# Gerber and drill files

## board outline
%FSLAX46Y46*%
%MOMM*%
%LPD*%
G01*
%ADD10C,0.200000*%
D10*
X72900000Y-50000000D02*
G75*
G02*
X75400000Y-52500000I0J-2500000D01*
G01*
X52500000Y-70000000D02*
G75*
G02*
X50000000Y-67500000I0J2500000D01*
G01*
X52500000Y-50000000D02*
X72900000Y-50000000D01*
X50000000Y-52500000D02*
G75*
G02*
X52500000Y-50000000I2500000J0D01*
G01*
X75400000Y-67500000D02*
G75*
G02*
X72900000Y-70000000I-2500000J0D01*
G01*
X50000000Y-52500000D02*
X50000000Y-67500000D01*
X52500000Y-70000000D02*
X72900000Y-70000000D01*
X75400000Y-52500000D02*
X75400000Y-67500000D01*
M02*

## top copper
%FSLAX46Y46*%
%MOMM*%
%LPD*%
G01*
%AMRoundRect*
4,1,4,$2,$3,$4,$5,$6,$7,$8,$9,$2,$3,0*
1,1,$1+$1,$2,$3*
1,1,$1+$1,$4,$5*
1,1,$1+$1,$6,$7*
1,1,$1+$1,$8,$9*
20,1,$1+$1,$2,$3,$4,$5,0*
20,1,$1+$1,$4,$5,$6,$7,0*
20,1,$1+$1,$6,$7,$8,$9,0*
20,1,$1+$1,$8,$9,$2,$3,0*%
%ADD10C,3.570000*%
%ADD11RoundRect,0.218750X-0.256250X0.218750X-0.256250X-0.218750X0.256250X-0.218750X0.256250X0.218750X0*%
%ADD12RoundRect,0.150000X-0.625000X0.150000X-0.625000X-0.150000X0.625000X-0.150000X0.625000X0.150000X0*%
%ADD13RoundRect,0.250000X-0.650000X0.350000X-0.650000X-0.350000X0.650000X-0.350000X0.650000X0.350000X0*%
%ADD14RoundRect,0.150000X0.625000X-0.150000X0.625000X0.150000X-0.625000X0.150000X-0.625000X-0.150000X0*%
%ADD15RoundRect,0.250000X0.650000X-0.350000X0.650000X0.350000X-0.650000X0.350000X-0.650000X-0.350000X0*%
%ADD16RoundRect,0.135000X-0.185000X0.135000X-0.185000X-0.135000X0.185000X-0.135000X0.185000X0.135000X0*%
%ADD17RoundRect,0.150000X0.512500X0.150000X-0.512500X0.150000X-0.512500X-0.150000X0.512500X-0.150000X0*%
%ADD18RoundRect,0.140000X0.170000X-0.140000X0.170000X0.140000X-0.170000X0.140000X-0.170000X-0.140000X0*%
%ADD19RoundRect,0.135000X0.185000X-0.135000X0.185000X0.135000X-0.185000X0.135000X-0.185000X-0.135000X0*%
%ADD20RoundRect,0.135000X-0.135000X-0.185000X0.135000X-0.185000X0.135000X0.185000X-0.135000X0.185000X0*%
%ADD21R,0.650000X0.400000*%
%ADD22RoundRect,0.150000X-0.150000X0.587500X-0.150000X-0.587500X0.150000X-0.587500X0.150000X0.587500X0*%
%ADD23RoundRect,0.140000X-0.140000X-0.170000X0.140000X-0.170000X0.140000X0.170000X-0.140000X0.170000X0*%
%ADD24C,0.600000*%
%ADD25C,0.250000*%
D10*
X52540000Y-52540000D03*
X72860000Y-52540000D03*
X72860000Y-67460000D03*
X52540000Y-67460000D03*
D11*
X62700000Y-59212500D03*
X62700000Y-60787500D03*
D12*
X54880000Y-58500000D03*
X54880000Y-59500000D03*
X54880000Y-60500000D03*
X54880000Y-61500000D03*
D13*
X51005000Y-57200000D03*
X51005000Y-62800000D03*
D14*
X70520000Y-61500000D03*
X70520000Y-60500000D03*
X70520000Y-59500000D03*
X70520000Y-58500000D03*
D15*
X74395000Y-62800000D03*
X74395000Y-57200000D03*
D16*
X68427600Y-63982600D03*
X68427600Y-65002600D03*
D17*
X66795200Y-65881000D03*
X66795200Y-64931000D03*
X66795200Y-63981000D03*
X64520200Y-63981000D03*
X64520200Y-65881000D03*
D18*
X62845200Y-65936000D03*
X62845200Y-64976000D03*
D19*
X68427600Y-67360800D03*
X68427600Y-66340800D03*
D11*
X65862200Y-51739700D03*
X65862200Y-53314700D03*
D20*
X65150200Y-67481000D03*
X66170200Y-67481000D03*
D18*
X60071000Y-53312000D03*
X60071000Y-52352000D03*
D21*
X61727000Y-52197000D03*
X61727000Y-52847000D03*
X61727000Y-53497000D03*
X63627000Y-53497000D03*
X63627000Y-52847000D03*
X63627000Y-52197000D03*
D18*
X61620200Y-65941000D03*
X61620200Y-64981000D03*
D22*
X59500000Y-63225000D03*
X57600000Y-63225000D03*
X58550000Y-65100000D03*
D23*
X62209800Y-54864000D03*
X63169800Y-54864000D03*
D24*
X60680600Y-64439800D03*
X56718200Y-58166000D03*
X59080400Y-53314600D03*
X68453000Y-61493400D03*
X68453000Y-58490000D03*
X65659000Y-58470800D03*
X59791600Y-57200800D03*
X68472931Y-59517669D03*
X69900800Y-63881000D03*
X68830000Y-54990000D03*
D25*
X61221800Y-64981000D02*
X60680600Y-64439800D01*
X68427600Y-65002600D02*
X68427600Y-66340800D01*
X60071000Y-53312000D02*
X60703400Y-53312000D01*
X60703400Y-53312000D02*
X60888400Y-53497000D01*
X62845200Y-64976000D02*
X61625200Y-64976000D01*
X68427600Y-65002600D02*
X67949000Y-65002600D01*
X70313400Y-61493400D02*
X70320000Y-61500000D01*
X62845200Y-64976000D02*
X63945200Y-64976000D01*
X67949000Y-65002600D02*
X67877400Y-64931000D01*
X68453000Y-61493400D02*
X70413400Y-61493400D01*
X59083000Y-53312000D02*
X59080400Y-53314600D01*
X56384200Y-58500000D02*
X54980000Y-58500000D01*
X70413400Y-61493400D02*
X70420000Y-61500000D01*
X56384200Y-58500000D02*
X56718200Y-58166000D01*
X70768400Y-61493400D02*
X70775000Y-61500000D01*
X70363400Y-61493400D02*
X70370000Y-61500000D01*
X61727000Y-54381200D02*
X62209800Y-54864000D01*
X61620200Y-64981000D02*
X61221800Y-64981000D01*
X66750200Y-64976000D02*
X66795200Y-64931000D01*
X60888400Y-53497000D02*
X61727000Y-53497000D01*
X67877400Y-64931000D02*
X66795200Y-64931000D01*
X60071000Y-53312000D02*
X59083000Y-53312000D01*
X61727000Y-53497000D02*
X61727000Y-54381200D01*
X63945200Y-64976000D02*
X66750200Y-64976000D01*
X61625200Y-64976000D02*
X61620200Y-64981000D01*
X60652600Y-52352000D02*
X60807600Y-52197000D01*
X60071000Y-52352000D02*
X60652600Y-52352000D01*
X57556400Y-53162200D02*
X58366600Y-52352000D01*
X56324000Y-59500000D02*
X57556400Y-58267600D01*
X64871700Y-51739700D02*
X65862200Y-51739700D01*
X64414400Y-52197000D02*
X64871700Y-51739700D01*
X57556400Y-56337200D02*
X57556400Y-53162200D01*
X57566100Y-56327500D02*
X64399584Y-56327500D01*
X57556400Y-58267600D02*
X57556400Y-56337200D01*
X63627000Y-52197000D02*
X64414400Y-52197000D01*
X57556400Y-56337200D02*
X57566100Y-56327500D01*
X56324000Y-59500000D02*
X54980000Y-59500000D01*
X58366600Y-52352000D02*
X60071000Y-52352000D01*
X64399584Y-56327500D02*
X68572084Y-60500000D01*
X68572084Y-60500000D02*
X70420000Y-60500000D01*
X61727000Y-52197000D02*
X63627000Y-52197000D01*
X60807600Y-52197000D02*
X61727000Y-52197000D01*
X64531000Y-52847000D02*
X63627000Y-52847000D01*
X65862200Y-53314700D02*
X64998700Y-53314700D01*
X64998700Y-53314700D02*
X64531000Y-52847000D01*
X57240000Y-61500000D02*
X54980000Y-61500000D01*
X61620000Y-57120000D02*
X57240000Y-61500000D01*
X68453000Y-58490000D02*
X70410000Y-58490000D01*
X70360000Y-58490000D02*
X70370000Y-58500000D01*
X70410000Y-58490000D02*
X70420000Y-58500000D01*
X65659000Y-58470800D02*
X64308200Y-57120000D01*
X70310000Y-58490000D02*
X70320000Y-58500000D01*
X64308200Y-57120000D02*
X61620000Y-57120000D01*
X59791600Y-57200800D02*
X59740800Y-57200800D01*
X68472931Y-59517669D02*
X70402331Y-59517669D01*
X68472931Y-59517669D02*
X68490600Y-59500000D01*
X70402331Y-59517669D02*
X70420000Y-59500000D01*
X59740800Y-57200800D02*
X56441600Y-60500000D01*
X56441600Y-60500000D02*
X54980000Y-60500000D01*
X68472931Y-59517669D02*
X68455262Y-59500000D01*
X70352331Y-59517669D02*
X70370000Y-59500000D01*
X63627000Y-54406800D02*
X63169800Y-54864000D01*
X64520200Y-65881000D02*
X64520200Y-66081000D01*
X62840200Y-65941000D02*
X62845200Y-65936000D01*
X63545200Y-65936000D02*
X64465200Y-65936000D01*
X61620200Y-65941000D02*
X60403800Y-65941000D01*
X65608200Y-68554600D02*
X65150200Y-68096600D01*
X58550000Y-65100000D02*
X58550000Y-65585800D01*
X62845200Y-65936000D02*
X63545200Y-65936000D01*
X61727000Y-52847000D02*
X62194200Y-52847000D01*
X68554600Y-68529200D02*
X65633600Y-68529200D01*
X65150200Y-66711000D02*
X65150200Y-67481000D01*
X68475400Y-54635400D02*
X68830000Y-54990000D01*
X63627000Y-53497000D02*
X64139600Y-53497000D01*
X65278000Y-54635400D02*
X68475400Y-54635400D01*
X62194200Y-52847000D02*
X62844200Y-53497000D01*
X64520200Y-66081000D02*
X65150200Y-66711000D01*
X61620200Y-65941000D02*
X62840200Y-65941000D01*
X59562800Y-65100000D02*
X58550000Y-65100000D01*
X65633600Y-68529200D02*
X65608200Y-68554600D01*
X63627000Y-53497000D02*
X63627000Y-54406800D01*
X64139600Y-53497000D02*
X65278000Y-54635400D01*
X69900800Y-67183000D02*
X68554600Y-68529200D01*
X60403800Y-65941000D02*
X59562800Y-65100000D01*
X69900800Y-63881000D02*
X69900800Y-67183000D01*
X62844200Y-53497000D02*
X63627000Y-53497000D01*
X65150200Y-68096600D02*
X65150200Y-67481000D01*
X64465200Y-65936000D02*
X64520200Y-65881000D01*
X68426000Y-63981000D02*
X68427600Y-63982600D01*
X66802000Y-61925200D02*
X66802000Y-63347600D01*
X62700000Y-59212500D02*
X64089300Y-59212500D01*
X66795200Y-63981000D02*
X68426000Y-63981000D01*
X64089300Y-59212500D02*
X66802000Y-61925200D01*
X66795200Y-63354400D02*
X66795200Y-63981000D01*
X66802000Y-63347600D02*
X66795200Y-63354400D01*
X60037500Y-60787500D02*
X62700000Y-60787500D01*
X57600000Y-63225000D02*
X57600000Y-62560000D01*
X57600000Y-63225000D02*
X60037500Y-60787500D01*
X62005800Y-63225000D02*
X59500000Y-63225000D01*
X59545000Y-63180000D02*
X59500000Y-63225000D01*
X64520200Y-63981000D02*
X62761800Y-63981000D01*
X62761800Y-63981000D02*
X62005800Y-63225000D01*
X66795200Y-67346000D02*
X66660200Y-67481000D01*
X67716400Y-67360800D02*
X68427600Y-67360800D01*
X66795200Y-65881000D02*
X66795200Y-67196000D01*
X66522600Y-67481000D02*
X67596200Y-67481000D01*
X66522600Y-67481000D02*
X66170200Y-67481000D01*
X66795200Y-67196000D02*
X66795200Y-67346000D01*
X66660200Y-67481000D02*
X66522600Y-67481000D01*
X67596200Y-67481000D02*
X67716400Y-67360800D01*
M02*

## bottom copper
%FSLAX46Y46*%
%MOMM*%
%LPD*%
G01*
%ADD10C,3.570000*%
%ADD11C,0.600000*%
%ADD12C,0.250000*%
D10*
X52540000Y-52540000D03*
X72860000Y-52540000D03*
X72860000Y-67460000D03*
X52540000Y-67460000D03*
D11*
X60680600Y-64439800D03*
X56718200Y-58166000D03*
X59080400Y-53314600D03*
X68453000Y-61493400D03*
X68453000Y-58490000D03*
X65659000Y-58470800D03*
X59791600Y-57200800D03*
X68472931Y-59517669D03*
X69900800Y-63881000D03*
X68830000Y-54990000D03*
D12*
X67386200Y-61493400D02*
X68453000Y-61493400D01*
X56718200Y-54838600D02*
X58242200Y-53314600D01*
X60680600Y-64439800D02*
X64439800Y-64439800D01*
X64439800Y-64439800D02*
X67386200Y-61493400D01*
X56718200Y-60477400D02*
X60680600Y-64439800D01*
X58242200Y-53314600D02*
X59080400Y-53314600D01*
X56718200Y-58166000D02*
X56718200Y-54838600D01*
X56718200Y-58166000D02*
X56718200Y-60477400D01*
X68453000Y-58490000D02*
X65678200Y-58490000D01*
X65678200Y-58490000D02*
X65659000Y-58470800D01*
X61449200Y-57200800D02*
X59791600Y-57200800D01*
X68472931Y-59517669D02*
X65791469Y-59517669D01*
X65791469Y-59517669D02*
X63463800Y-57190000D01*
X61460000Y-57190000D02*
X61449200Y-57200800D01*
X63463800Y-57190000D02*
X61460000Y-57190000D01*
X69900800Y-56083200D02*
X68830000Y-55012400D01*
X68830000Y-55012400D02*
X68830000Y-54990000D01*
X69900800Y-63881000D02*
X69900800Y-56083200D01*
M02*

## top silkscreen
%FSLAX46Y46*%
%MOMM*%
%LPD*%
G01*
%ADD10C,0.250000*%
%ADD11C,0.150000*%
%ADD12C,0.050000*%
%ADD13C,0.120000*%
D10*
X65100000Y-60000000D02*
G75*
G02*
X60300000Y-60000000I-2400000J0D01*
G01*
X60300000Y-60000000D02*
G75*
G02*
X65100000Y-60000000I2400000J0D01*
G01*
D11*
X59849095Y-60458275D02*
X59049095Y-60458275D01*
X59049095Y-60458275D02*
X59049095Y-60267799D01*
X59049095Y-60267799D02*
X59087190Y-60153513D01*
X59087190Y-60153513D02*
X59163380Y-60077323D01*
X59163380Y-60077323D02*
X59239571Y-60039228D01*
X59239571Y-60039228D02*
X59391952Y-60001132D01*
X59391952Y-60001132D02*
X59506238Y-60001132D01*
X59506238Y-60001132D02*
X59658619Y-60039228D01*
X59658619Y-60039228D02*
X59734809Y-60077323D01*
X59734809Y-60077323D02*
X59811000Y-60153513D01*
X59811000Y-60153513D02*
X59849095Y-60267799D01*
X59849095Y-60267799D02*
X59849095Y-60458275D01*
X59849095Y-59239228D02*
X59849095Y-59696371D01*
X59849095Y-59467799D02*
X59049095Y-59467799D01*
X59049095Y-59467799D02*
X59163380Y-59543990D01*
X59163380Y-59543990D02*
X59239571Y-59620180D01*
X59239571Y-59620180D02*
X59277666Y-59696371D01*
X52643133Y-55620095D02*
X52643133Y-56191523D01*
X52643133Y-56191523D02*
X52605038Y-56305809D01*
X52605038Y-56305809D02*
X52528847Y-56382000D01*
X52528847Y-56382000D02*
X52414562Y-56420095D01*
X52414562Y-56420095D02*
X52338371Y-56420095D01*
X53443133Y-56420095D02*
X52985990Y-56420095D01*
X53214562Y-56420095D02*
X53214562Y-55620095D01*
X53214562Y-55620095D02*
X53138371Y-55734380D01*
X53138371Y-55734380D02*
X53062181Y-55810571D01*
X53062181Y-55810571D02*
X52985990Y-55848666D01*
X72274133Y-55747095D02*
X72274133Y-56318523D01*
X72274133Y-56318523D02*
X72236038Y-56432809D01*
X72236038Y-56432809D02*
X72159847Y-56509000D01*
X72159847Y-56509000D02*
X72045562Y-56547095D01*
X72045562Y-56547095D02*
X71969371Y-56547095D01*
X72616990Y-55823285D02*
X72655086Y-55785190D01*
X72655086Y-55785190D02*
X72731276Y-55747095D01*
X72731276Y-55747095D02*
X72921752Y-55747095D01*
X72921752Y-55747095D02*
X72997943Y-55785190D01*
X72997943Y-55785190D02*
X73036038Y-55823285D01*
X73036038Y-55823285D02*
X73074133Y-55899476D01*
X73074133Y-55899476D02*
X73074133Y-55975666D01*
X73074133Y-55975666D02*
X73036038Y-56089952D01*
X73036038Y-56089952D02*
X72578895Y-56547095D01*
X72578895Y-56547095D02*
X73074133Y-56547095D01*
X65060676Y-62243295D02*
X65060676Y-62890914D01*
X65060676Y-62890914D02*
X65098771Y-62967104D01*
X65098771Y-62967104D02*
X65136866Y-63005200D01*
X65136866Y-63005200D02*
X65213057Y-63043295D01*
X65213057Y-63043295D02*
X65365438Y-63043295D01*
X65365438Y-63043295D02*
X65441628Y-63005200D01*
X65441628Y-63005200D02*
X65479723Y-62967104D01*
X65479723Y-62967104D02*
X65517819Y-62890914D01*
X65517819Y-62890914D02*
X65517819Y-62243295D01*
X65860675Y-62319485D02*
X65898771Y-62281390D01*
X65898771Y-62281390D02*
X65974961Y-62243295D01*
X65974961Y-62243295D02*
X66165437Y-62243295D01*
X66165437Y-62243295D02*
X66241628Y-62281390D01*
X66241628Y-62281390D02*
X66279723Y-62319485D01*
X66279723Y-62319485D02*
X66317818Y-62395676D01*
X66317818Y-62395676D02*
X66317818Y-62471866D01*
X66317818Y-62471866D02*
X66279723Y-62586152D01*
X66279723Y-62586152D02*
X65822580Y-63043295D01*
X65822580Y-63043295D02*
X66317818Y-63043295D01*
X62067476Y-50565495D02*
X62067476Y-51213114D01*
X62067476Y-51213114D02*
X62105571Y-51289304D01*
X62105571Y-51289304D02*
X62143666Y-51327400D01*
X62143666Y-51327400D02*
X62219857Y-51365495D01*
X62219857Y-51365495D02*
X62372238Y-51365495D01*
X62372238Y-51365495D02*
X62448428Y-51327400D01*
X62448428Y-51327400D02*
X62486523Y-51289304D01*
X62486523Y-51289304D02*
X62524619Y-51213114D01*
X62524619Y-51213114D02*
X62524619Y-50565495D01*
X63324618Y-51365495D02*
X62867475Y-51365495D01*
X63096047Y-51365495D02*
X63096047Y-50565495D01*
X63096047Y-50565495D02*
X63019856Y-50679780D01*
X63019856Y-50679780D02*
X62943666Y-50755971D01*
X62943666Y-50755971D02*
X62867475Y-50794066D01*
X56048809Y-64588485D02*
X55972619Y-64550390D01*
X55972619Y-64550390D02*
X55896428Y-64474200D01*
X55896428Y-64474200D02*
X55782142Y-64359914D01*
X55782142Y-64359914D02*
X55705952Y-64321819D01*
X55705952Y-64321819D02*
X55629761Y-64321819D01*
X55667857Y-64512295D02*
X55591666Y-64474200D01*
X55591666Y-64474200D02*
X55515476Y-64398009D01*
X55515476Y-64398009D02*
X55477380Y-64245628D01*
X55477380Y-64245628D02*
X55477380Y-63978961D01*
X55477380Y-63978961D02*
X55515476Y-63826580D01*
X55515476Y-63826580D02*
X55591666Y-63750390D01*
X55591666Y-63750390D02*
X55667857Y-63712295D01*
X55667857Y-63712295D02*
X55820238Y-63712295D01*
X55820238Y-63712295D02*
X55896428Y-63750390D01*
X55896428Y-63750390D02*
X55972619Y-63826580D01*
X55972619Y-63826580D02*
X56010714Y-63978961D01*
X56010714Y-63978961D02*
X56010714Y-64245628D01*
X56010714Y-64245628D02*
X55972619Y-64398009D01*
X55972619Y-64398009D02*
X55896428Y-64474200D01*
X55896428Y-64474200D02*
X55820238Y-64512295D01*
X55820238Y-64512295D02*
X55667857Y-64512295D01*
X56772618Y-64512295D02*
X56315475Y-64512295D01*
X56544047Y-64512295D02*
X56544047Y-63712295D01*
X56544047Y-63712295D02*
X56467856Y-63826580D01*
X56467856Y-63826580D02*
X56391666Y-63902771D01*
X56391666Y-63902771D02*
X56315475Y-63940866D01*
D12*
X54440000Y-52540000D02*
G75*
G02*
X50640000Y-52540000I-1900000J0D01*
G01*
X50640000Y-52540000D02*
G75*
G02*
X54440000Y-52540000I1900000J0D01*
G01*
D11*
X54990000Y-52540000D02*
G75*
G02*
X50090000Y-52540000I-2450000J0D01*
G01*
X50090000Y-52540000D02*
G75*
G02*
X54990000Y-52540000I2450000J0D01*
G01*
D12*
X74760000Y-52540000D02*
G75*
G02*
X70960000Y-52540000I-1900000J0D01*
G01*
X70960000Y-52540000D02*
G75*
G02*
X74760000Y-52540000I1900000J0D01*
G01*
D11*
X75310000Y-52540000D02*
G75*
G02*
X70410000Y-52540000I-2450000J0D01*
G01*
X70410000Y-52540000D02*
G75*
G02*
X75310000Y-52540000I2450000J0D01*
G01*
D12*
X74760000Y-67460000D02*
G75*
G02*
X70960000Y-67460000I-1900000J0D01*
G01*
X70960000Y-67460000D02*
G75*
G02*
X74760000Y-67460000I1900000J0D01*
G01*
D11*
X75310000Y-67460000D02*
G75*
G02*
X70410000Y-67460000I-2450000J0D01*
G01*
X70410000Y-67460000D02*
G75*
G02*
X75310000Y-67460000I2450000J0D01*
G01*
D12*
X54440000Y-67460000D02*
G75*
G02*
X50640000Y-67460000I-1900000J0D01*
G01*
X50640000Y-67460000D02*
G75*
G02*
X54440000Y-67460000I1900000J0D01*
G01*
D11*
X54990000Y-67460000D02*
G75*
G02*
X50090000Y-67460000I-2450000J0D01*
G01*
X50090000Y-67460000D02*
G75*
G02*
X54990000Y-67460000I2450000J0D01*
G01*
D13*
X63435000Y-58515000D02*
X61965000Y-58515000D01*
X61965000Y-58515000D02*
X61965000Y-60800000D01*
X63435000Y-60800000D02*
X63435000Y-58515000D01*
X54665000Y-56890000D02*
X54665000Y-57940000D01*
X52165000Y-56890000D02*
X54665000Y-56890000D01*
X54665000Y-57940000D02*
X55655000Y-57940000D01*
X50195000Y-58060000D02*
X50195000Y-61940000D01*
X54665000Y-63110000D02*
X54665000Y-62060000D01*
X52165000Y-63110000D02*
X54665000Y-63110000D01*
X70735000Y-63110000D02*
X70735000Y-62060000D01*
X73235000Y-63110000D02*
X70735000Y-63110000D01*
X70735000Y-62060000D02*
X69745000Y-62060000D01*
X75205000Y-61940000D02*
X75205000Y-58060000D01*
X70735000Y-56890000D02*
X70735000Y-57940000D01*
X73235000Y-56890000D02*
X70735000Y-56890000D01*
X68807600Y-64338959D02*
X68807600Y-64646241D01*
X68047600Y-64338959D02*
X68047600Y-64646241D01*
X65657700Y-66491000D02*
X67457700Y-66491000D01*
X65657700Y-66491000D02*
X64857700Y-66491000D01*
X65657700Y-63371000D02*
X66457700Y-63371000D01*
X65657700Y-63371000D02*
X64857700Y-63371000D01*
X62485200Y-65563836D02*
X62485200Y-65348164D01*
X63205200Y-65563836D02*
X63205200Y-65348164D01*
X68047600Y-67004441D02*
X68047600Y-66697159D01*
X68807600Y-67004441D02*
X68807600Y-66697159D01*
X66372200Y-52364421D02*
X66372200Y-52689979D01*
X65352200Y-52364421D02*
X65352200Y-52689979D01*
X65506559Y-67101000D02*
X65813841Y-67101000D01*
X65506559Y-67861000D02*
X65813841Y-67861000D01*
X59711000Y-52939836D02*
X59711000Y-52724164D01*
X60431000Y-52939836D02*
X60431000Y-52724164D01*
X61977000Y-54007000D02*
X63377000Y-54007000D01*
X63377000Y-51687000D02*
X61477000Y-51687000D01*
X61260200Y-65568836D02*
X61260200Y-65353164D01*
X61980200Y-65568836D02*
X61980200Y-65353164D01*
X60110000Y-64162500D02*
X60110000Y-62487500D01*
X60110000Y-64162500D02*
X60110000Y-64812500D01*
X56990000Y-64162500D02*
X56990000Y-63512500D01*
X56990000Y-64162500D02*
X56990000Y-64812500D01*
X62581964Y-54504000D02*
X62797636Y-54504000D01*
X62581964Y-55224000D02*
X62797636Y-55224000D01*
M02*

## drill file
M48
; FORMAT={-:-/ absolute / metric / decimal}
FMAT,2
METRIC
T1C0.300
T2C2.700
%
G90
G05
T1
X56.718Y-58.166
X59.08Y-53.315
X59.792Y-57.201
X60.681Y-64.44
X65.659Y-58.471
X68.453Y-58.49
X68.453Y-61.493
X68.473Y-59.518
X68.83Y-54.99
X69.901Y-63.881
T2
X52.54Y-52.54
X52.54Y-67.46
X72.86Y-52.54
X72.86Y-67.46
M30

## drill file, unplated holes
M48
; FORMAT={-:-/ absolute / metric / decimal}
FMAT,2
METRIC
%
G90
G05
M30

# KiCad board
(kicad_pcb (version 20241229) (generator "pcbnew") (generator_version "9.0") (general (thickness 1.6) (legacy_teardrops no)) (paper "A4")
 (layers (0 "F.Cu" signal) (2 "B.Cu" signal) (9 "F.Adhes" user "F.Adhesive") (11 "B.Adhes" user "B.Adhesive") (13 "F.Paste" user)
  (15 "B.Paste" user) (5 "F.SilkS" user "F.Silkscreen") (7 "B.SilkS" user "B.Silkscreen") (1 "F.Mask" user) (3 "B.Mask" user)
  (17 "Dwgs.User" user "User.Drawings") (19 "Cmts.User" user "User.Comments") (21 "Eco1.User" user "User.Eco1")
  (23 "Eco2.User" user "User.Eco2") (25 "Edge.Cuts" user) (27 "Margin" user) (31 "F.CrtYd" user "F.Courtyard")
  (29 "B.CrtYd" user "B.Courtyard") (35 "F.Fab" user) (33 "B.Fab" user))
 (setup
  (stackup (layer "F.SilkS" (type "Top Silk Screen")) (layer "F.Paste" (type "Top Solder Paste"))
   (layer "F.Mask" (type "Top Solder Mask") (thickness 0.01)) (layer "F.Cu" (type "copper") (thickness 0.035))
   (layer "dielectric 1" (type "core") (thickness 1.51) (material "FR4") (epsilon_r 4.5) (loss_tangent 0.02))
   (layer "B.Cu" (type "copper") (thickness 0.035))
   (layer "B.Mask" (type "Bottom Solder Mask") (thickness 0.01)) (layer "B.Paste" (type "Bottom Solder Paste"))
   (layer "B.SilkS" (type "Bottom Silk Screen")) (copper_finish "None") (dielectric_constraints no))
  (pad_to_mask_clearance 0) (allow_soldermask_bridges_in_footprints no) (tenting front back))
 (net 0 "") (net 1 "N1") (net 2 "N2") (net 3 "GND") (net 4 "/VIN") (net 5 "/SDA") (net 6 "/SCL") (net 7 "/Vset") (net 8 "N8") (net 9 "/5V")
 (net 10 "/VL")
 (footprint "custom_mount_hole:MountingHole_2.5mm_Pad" (layer "F.Cu") (at 52.54 52.54)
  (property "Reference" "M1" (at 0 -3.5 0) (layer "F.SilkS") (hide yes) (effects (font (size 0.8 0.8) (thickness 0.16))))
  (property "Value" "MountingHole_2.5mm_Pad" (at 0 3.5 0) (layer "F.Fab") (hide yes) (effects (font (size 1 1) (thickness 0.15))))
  (fp_circle (center 0 0) (end 1.9 0) (stroke (width 0.05) (type solid)) (fill no) (layer "F.SilkS"))
  (fp_circle (center 0 0) (end 2.45 0) (stroke (width 0.15) (type solid)) (fill no) (layer "F.SilkS"))
  (pad "~" thru_hole circle (at 0 0) (size 3.57 3.57) (drill 2.7) (layers "*.Cu" "*.Mask") (remove_unused_layers no)))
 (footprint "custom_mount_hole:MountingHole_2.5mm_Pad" (layer "F.Cu") (at 72.86 52.54)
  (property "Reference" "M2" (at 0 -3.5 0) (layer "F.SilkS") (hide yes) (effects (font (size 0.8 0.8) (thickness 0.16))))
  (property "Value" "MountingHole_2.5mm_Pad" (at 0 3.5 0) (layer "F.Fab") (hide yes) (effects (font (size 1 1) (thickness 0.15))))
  (fp_circle (center 0 0) (end 1.9 0) (stroke (width 0.05) (type solid)) (fill no) (layer "F.SilkS"))
  (fp_circle (center 0 0) (end 2.45 0) (stroke (width 0.15) (type solid)) (fill no) (layer "F.SilkS"))
  (pad "~" thru_hole circle (at 0 0) (size 3.57 3.57) (drill 2.7) (layers "*.Cu" "*.Mask") (remove_unused_layers no)))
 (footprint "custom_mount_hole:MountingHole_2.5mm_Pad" (layer "F.Cu") (at 72.86 67.46)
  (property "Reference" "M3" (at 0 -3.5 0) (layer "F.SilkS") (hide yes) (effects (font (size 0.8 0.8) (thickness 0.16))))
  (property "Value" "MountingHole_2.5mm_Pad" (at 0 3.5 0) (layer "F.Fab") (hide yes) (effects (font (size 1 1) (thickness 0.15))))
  (fp_circle (center 0 0) (end 1.9 0) (stroke (width 0.05) (type solid)) (fill no) (layer "F.SilkS"))
  (fp_circle (center 0 0) (end 2.45 0) (stroke (width 0.15) (type solid)) (fill no) (layer "F.SilkS"))
  (pad "~" thru_hole circle (at 0 0) (size 3.57 3.57) (drill 2.7) (layers "*.Cu" "*.Mask") (remove_unused_layers no)))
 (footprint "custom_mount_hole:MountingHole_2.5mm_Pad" (layer "F.Cu") (at 52.54 67.46)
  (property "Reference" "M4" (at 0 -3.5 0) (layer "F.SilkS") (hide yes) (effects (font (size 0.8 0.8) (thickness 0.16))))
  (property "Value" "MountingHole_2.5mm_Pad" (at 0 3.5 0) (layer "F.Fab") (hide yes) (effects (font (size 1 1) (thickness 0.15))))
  (fp_circle (center 0 0) (end 1.9 0) (stroke (width 0.05) (type solid)) (fill no) (layer "F.SilkS"))
  (fp_circle (center 0 0) (end 2.45 0) (stroke (width 0.15) (type solid)) (fill no) (layer "F.SilkS"))
  (pad "~" thru_hole circle (at 0 0) (size 3.57 3.57) (drill 2.7) (layers "*.Cu" "*.Mask") (remove_unused_layers no)))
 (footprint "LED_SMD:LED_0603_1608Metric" (layer "F.Cu") (at 62.7 60 -90)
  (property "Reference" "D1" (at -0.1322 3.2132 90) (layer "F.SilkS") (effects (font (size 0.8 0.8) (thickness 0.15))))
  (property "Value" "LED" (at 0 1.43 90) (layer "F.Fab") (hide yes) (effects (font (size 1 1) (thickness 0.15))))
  (fp_line (start -1.485 0.735) (end 0.8 0.735) (stroke (width 0.12) (type solid)) (layer "F.SilkS"))
  (fp_line (start -1.485 -0.735) (end -1.485 0.735) (stroke (width 0.12) (type solid)) (layer "F.SilkS"))
  (fp_line (start 0.8 -0.735) (end -1.485 -0.735) (stroke (width 0.12) (type solid)) (layer "F.SilkS"))
  (pad "1" smd roundrect (at -0.7875 0 270) (size 0.875 0.95) (layers "F.Cu" "F.Mask" "F.Paste") (roundrect_rratio 0.25) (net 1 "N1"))
  (pad "2" smd roundrect (at 0.7875 0 270) (size 0.875 0.95) (layers "F.Cu" "F.Mask" "F.Paste") (roundrect_rratio 0.25) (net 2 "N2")))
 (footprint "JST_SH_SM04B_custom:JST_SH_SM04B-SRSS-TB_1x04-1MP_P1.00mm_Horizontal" (layer "F.Cu") (at 52.88 60 -90)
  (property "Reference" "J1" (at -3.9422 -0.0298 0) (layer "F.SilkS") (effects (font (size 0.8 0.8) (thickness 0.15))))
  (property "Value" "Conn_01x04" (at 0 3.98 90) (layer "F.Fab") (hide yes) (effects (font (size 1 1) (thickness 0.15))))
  (fp_line (start -1.94 2.685) (end 1.94 2.685) (stroke (width 0.12) (type solid)) (layer "F.SilkS"))
  (fp_line (start -3.11 0.715) (end -3.11 -1.785) (stroke (width 0.12) (type solid)) (layer "F.SilkS"))
  (fp_line (start 3.11 0.715) (end 3.11 -1.785) (stroke (width 0.12) (type solid)) (layer "F.SilkS"))
  (fp_line (start -3.11 -1.785) (end -2.06 -1.785) (stroke (width 0.12) (type solid)) (layer "F.SilkS"))
  (fp_line (start -2.06 -1.785) (end -2.06 -2.775) (stroke (width 0.12) (type solid)) (layer "F.SilkS"))
  (fp_line (start 3.11 -1.785) (end 2.06 -1.785) (stroke (width 0.12) (type solid)) (layer "F.SilkS"))
  (pad "1" smd roundrect (at -1.5 -2 270) (size 0.6 1.55) (layers "F.Cu" "F.Mask" "F.Paste") (roundrect_rratio 0.25) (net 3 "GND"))
  (pad "2" smd roundrect (at -0.5 -2 270) (size 0.6 1.55) (layers "F.Cu" "F.Mask" "F.Paste") (roundrect_rratio 0.25) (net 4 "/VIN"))
  (pad "3" smd roundrect (at 0.5 -2 270) (size 0.6 1.55) (layers "F.Cu" "F.Mask" "F.Paste") (roundrect_rratio 0.25) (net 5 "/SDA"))
  (pad "4" smd roundrect (at 1.5 -2 270) (size 0.6 1.55) (layers "F.Cu" "F.Mask" "F.Paste") (roundrect_rratio 0.25) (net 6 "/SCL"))
  (pad "MP" smd roundrect (at -2.8 1.875 270) (size 1.2 1.8) (layers "F.Cu" "F.Mask" "F.Paste") (roundrect_rratio 0.2083333333))
  (pad "MP" smd roundrect (at 2.8 1.875 270) (size 1.2 1.8) (layers "F.Cu" "F.Mask" "F.Paste") (roundrect_rratio 0.2083333333)))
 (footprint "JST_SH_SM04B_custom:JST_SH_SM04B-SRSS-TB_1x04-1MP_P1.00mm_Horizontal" (layer "F.Cu") (at 72.52 60 90)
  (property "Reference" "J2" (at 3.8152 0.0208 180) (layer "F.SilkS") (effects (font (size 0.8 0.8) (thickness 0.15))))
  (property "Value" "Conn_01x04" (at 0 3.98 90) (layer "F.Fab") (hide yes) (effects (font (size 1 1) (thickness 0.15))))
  (fp_line (start 3.11 -1.785) (end 2.06 -1.785) (stroke (width 0.12) (type solid)) (layer "F.SilkS"))
  (fp_line (start -2.06 -1.785) (end -2.06 -2.775) (stroke (width 0.12) (type solid)) (layer "F.SilkS"))
  (fp_line (start -3.11 -1.785) (end -2.06 -1.785) (stroke (width 0.12) (type solid)) (layer "F.SilkS"))
  (fp_line (start 3.11 0.715) (end 3.11 -1.785) (stroke (width 0.12) (type solid)) (layer "F.SilkS"))
  (fp_line (start -3.11 0.715) (end -3.11 -1.785) (stroke (width 0.12) (type solid)) (layer "F.SilkS"))
  (fp_line (start -1.94 2.685) (end 1.94 2.685) (stroke (width 0.12) (type solid)) (layer "F.SilkS"))
  (pad "1" smd roundrect (at -1.5 -2 90) (size 0.6 1.55) (layers "F.Cu" "F.Mask" "F.Paste") (roundrect_rratio 0.25) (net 3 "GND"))
  (pad "2" smd roundrect (at -0.5 -2 90) (size 0.6 1.55) (layers "F.Cu" "F.Mask" "F.Paste") (roundrect_rratio 0.25) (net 4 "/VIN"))
  (pad "3" smd roundrect (at 0.5 -2 90) (size 0.6 1.55) (layers "F.Cu" "F.Mask" "F.Paste") (roundrect_rratio 0.25) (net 5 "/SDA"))
  (pad "4" smd roundrect (at 1.5 -2 90) (size 0.6 1.55) (layers "F.Cu" "F.Mask" "F.Paste") (roundrect_rratio 0.25) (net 6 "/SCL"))
  (pad "MP" smd roundrect (at -2.8 1.875 90) (size 1.2 1.8) (layers "F.Cu" "F.Mask" "F.Paste") (roundrect_rratio 0.2083333333))
  (pad "MP" smd roundrect (at 2.8 1.875 90) (size 1.2 1.8) (layers "F.Cu" "F.Mask" "F.Paste") (roundrect_rratio 0.2083333333)))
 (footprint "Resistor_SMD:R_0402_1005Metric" (layer "F.Cu") (at 68.4276 64.4926 -90)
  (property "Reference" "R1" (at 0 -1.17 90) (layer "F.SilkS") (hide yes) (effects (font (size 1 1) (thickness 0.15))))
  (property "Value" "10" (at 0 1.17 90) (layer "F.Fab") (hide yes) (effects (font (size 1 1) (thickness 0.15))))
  (fp_line (start -0.153641 0.38) (end 0.153641 0.38) (stroke (width 0.12) (type solid)) (layer "F.SilkS"))
  (fp_line (start -0.153641 -0.38) (end 0.153641 -0.38) (stroke (width 0.12) (type solid)) (layer "F.SilkS"))
  (pad "1" smd roundrect (at -0.51 0 270) (size 0.54 0.64) (layers "F.Cu" "F.Mask" "F.Paste") (roundrect_rratio 0.25) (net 1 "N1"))
  (pad "2" smd roundrect (at 0.51 0 270) (size 0.54 0.64) (layers "F.Cu" "F.Mask" "F.Paste") (roundrect_rratio 0.25) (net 3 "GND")))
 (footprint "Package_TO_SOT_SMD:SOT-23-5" (layer "F.Cu") (at 65.6577 64.931 180)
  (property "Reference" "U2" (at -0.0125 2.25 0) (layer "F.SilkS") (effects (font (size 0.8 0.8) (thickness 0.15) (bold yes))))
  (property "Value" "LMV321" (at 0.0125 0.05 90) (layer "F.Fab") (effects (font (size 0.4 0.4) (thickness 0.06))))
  (fp_line (start 0 1.56) (end 0.8 1.56) (stroke (width 0.12) (type solid)) (layer "F.SilkS"))
  (fp_line (start 0 1.56) (end -0.8 1.56) (stroke (width 0.12) (type solid)) (layer "F.SilkS"))
  (fp_line (start 0 -1.56) (end 0.8 -1.56) (stroke (width 0.12) (type solid)) (layer "F.SilkS"))
  (fp_line (start 0 -1.56) (end -1.8 -1.56) (stroke (width 0.12) (type solid)) (layer "F.SilkS"))
  (pad "1" smd roundrect (at -1.1375 -0.95 180) (size 1.325 0.6) (layers "F.Cu" "F.Mask" "F.Paste") (roundrect_rratio 0.25) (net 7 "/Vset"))
  (pad "2" smd roundrect (at -1.1375 0 180) (size 1.325 0.6) (layers "F.Cu" "F.Mask" "F.Paste") (roundrect_rratio 0.25) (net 3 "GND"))
  (pad "3" smd roundrect (at -1.1375 0.95 180) (size 1.325 0.6) (layers "F.Cu" "F.Mask" "F.Paste") (roundrect_rratio 0.25) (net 1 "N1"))
  (pad "4" smd roundrect (at 1.1375 0.95 180) (size 1.325 0.6) (layers "F.Cu" "F.Mask" "F.Paste") (roundrect_rratio 0.25) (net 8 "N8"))
  (pad "5" smd roundrect (at 1.1375 -0.95 180) (size 1.325 0.6) (layers "F.Cu" "F.Mask" "F.Paste") (roundrect_rratio 0.25) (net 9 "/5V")))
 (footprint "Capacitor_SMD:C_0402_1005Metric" (layer "F.Cu") (at 62.8452 65.456 90)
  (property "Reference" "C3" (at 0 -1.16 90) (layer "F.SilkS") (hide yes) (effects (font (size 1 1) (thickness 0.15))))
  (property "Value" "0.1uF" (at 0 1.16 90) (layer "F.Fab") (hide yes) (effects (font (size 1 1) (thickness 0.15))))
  (fp_line (start -0.107836 -0.36) (end 0.107836 -0.36) (stroke (width 0.12) (type solid)) (layer "F.SilkS"))
  (fp_line (start -0.107836 0.36) (end 0.107836 0.36) (stroke (width 0.12) (type solid)) (layer "F.SilkS"))
  (pad "1" smd roundrect (at -0.48 0 90) (size 0.56 0.62) (layers "F.Cu" "F.Mask" "F.Paste") (roundrect_rratio 0.25) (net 9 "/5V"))
  (pad "2" smd roundrect (at 0.48 0 90) (size 0.56 0.62) (layers "F.Cu" "F.Mask" "F.Paste") (roundrect_rratio 0.25) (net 3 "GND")))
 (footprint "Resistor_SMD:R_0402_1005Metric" (layer "F.Cu") (at 68.4276 66.8508 90)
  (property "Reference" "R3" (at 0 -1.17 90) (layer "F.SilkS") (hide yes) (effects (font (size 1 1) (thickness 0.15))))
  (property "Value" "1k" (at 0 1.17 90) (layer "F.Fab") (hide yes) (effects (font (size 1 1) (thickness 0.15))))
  (fp_line (start -0.153641 -0.38) (end 0.153641 -0.38) (stroke (width 0.12) (type solid)) (layer "F.SilkS"))
  (fp_line (start -0.153641 0.38) (end 0.153641 0.38) (stroke (width 0.12) (type solid)) (layer "F.SilkS"))
  (pad "1" smd roundrect (at -0.51 0 90) (size 0.54 0.64) (layers "F.Cu" "F.Mask" "F.Paste") (roundrect_rratio 0.25) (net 7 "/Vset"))
  (pad "2" smd roundrect (at 0.51 0 90) (size 0.54 0.64) (layers "F.Cu" "F.Mask" "F.Paste") (roundrect_rratio 0.25) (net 3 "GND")))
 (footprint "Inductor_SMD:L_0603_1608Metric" (layer "F.Cu") (at 65.8622 52.5272 -90)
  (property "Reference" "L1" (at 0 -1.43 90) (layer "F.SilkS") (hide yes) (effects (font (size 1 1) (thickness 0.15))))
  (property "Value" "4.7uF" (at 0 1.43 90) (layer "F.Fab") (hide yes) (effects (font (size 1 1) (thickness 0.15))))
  (fp_line (start -0.162779 0.51) (end 0.162779 0.51) (stroke (width 0.12) (type solid)) (layer "F.SilkS"))
  (fp_line (start -0.162779 -0.51) (end 0.162779 -0.51) (stroke (width 0.12) (type solid)) (layer "F.SilkS"))
  (pad "1" smd roundrect (at -0.7875 0 270) (size 0.875 0.95) (layers "F.Cu" "F.Mask" "F.Paste") (roundrect_rratio 0.25) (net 4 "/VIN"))
  (pad "2" smd roundrect (at 0.7875 0 270) (size 0.875 0.95) (layers "F.Cu" "F.Mask" "F.Paste") (roundrect_rratio 0.25) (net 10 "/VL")))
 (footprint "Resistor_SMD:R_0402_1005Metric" (layer "F.Cu") (at 65.6602 67.481)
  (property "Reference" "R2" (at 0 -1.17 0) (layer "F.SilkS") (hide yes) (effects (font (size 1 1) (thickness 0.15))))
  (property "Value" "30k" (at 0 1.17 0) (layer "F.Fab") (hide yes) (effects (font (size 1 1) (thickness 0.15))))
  (fp_line (start -0.153641 -0.38) (end 0.153641 -0.38) (stroke (width 0.12) (type solid)) (layer "F.SilkS"))
  (fp_line (start -0.153641 0.38) (end 0.153641 0.38) (stroke (width 0.12) (type solid)) (layer "F.SilkS"))
  (pad "1" smd roundrect (at -0.51 0) (size 0.54 0.64) (layers "F.Cu" "F.Mask" "F.Paste") (roundrect_rratio 0.25) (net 9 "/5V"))
  (pad "2" smd roundrect (at 0.51 0) (size 0.54 0.64) (layers "F.Cu" "F.Mask" "F.Paste") (roundrect_rratio 0.25) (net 7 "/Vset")))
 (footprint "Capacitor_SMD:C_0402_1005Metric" (layer "F.Cu") (at 60.071 52.832 90)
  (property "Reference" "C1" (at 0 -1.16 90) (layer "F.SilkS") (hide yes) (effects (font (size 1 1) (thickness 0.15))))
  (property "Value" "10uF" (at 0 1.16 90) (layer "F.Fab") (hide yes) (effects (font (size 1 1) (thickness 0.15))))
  (fp_line (start -0.107836 -0.36) (end 0.107836 -0.36) (stroke (width 0.12) (type solid)) (layer "F.SilkS"))
  (fp_line (start -0.107836 0.36) (end 0.107836 0.36) (stroke (width 0.12) (type solid)) (layer "F.SilkS"))
  (pad "1" smd roundrect (at -0.48 0 90) (size 0.56 0.62) (layers "F.Cu" "F.Mask" "F.Paste") (roundrect_rratio 0.25) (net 3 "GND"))
  (pad "2" smd roundrect (at 0.48 0 90) (size 0.56 0.62) (layers "F.Cu" "F.Mask" "F.Paste") (roundrect_rratio 0.25) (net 4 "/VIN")))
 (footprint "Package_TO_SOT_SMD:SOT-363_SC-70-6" (layer "F.Cu") (at 62.677 52.847)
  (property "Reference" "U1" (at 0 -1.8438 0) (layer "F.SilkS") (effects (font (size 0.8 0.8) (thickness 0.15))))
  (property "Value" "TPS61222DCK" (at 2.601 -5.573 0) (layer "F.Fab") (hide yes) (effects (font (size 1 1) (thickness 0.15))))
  (fp_line (start -0.7 1.16) (end 0.7 1.16) (stroke (width 0.12) (type solid)) (layer "F.SilkS"))
  (fp_line (start 0.7 -1.16) (end -1.2 -1.16) (stroke (width 0.12) (type solid)) (layer "F.SilkS"))
  (pad "1" smd rect (at -0.95 -0.65) (size 0.65 0.4) (layers "F.Cu" "F.Mask" "F.Paste") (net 4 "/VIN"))
  (pad "2" smd rect (at -0.95 0) (size 0.65 0.4) (layers "F.Cu" "F.Mask" "F.Paste") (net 9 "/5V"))
  (pad "3" smd rect (at -0.95 0.65) (size 0.65 0.4) (layers "F.Cu" "F.Mask" "F.Paste") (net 3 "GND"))
  (pad "4" smd rect (at 0.95 0.65) (size 0.65 0.4) (layers "F.Cu" "F.Mask" "F.Paste") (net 9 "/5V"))
  (pad "5" smd rect (at 0.95 0) (size 0.65 0.4) (layers "F.Cu" "F.Mask" "F.Paste") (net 10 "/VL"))
  (pad "6" smd rect (at 0.95 -0.65) (size 0.65 0.4) (layers "F.Cu" "F.Mask" "F.Paste") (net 4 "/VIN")))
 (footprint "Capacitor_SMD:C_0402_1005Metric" (layer "F.Cu") (at 61.6202 65.461 90)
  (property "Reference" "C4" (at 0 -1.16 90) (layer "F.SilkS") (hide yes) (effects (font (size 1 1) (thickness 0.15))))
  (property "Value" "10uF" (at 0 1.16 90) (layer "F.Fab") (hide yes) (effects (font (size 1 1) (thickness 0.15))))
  (fp_line (start -0.107836 -0.36) (end 0.107836 -0.36) (stroke (width 0.12) (type solid)) (layer "F.SilkS"))
  (fp_line (start -0.107836 0.36) (end 0.107836 0.36) (stroke (width 0.12) (type solid)) (layer "F.SilkS"))
  (pad "1" smd roundrect (at -0.48 0 90) (size 0.56 0.62) (layers "F.Cu" "F.Mask" "F.Paste") (roundrect_rratio 0.25) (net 9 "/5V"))
  (pad "2" smd roundrect (at 0.48 0 90) (size 0.56 0.62) (layers "F.Cu" "F.Mask" "F.Paste") (roundrect_rratio 0.25) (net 3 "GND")))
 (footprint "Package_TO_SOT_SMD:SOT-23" (layer "F.Cu") (at 58.55 64.1625 -90)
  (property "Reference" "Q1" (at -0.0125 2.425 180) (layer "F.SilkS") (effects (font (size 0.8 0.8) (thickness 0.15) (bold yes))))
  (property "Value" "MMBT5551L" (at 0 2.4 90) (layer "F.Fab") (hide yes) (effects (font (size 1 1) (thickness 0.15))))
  (fp_line (start 0 1.56) (end -0.65 1.56) (stroke (width 0.12) (type solid)) (layer "F.SilkS"))
  (fp_line (start 0 1.56) (end 0.65 1.56) (stroke (width 0.12) (type solid)) (layer "F.SilkS"))
  (fp_line (start 0 -1.56) (end -1.675 -1.56) (stroke (width 0.12) (type solid)) (layer "F.SilkS"))
  (fp_line (start 0 -1.56) (end 0.65 -1.56) (stroke (width 0.12) (type solid)) (layer "F.SilkS"))
  (pad "1" smd roundrect (at -0.9375 -0.95 270) (size 1.475 0.6) (layers "F.Cu" "F.Mask" "F.Paste") (roundrect_rratio 0.25) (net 8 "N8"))
  (pad "2" smd roundrect (at -0.9375 0.95 270) (size 1.475 0.6) (layers "F.Cu" "F.Mask" "F.Paste") (roundrect_rratio 0.25) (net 2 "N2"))
  (pad "3" smd roundrect (at 0.9375 0 270) (size 1.475 0.6) (layers "F.Cu" "F.Mask" "F.Paste") (roundrect_rratio 0.25) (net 9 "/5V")))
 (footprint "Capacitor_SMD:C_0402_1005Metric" (layer "F.Cu") (at 62.6898 54.864)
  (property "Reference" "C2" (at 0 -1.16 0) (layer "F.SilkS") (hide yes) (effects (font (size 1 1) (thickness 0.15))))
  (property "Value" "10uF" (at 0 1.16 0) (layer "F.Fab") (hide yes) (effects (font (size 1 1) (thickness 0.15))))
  (fp_line (start -0.107836 -0.36) (end 0.107836 -0.36) (stroke (width 0.12) (type solid)) (layer "F.SilkS"))
  (fp_line (start -0.107836 0.36) (end 0.107836 0.36) (stroke (width 0.12) (type solid)) (layer "F.SilkS"))
  (pad "1" smd roundrect (at -0.48 0) (size 0.56 0.62) (layers "F.Cu" "F.Mask" "F.Paste") (roundrect_rratio 0.25) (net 3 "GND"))
  (pad "2" smd roundrect (at 0.48 0) (size 0.56 0.62) (layers "F.Cu" "F.Mask" "F.Paste") (roundrect_rratio 0.25) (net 9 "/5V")))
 (gr_circle (center 62.7 60) (end 65.1 60) (stroke (width 0.25) (type solid)) (fill no) (layer "F.SilkS"))
 (gr_arc (start 72.9 50) (mid 74.667767 50.732233) (end 75.4 52.5) (stroke (width 0.2) (type solid)) (layer "Edge.Cuts"))
 (gr_arc (start 52.5 70) (mid 50.732233 69.267767) (end 50 67.5) (stroke (width 0.2) (type solid)) (layer "Edge.Cuts"))
 (gr_line (start 52.5 50) (end 72.9 50) (stroke (width 0.2) (type solid)) (layer "Edge.Cuts"))
 (gr_arc (start 50 52.5) (mid 50.732233 50.732233) (end 52.5 50) (stroke (width 0.2) (type solid)) (layer "Edge.Cuts"))
 (gr_arc (start 75.4 67.5) (mid 74.667767 69.267767) (end 72.9 70) (stroke (width 0.2) (type solid)) (layer "Edge.Cuts"))
 (gr_line (start 50 52.5) (end 50 67.5) (stroke (width 0.2) (type solid)) (layer "Edge.Cuts"))
 (gr_line (start 52.5 70) (end 72.9 70) (stroke (width 0.2) (type solid)) (layer "Edge.Cuts"))
 (gr_line (start 75.4 52.5) (end 75.4 67.5) (stroke (width 0.2) (type solid)) (layer "Edge.Cuts"))
 (segment (start 61.2218 64.981) (end 60.6806 64.4398) (width 0.25) (layer "F.Cu") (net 3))
 (segment (start 68.4276 65.0026) (end 68.4276 66.3408) (width 0.25) (layer "F.Cu") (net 3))
 (segment (start 60.071 53.312) (end 60.7034 53.312) (width 0.25) (layer "F.Cu") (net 3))
 (segment (start 60.7034 53.312) (end 60.8884 53.497) (width 0.25) (layer "F.Cu") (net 3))
 (segment (start 62.8452 64.976) (end 61.6252 64.976) (width 0.25) (layer "F.Cu") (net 3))
 (segment (start 68.4276 65.0026) (end 67.949 65.0026) (width 0.25) (layer "F.Cu") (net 3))
 (segment (start 70.3134 61.4934) (end 70.32 61.5) (width 0.25) (layer "F.Cu") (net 3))
 (segment (start 62.8452 64.976) (end 63.9452 64.976) (width 0.25) (layer "F.Cu") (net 3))
 (segment (start 67.949 65.0026) (end 67.8774 64.931) (width 0.25) (layer "F.Cu") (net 3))
 (segment (start 68.453 61.4934) (end 70.4134 61.4934) (width 0.25) (layer "F.Cu") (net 3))
 (segment (start 59.083 53.312) (end 59.0804 53.3146) (width 0.25) (layer "F.Cu") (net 3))
 (segment (start 56.3842 58.5) (end 54.98 58.5) (width 0.25) (layer "F.Cu") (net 3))
 (segment (start 70.4134 61.4934) (end 70.42 61.5) (width 0.25) (layer "F.Cu") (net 3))
 (segment (start 56.3842 58.5) (end 56.7182 58.166) (width 0.25) (layer "F.Cu") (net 3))
 (segment (start 70.7684 61.4934) (end 70.775 61.5) (width 0.25) (layer "F.Cu") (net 3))
 (segment (start 70.3634 61.4934) (end 70.37 61.5) (width 0.25) (layer "F.Cu") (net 3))
 (segment (start 61.727 54.3812) (end 62.2098 54.864) (width 0.25) (layer "F.Cu") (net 3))
 (segment (start 61.6202 64.981) (end 61.2218 64.981) (width 0.25) (layer "F.Cu") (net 3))
 (segment (start 66.7502 64.976) (end 66.7952 64.931) (width 0.25) (layer "F.Cu") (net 3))
 (segment (start 60.8884 53.497) (end 61.727 53.497) (width 0.25) (layer "F.Cu") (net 3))
 (segment (start 67.8774 64.931) (end 66.7952 64.931) (width 0.25) (layer "F.Cu") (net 3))
 (segment (start 60.071 53.312) (end 59.083 53.312) (width 0.25) (layer "F.Cu") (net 3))
 (segment (start 61.727 53.497) (end 61.727 54.3812) (width 0.25) (layer "F.Cu") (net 3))
 (segment (start 63.9452 64.976) (end 66.7502 64.976) (width 0.25) (layer "F.Cu") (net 3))
 (segment (start 61.6252 64.976) (end 61.6202 64.981) (width 0.25) (layer "F.Cu") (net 3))
 (via (at 60.6806 64.4398) (size 0.6) (drill 0.3) (layers "F.Cu" "B.Cu") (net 3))
 (via (at 56.7182 58.166) (size 0.6) (drill 0.3) (layers "F.Cu" "B.Cu") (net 3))
 (via (at 59.0804 53.3146) (size 0.6) (drill 0.3) (layers "F.Cu" "B.Cu") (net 3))
 (via (at 68.453 61.4934) (size 0.6) (drill 0.3) (layers "F.Cu" "B.Cu") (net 3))
 (segment (start 67.3862 61.4934) (end 68.453 61.4934) (width 0.25) (layer "B.Cu") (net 3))
 (segment (start 56.7182 54.8386) (end 58.2422 53.3146) (width 0.25) (layer "B.Cu") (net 3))
 (segment (start 60.6806 64.4398) (end 64.4398 64.4398) (width 0.25) (layer "B.Cu") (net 3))
 (segment (start 64.4398 64.4398) (end 67.3862 61.4934) (width 0.25) (layer "B.Cu") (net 3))
 (segment (start 56.7182 60.4774) (end 60.6806 64.4398) (width 0.25) (layer "B.Cu") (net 3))
 (segment (start 58.2422 53.3146) (end 59.0804 53.3146) (width 0.25) (layer "B.Cu") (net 3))
 (segment (start 56.7182 58.166) (end 56.7182 54.8386) (width 0.25) (layer "B.Cu") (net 3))
 (segment (start 56.7182 58.166) (end 56.7182 60.4774) (width 0.25) (layer "B.Cu") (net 3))
 (segment (start 60.6526 52.352) (end 60.8076 52.197) (width 0.25) (layer "F.Cu") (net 4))
 (segment (start 60.071 52.352) (end 60.6526 52.352) (width 0.25) (layer "F.Cu") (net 4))
 (segment (start 57.5564 53.1622) (end 58.3666 52.352) (width 0.25) (layer "F.Cu") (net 4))
 (segment (start 56.324 59.5) (end 57.5564 58.2676) (width 0.25) (layer "F.Cu") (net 4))
 (segment (start 64.8717 51.7397) (end 65.8622 51.7397) (width 0.25) (layer "F.Cu") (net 4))
 (segment (start 64.4144 52.197) (end 64.8717 51.7397) (width 0.25) (layer "F.Cu") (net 4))
 (segment (start 57.5564 56.3372) (end 57.5564 53.1622) (width 0.25) (layer "F.Cu") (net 4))
 (segment (start 57.5661 56.3275) (end 64.399584 56.3275) (width 0.25) (layer "F.Cu") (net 4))
 (segment (start 57.5564 58.2676) (end 57.5564 56.3372) (width 0.25) (layer "F.Cu") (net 4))
 (segment (start 63.627 52.197) (end 64.4144 52.197) (width 0.25) (layer "F.Cu") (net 4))
 (segment (start 57.5564 56.3372) (end 57.5661 56.3275) (width 0.25) (layer "F.Cu") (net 4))
 (segment (start 56.324 59.5) (end 54.98 59.5) (width 0.25) (layer "F.Cu") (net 4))
 (segment (start 58.3666 52.352) (end 60.071 52.352) (width 0.25) (layer "F.Cu") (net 4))
 (segment (start 64.399584 56.3275) (end 68.572084 60.5) (width 0.25) (layer "F.Cu") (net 4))
 (segment (start 68.572084 60.5) (end 70.42 60.5) (width 0.25) (layer "F.Cu") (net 4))
 (segment (start 61.727 52.197) (end 63.627 52.197) (width 0.25) (layer "F.Cu") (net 4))
 (segment (start 60.8076 52.197) (end 61.727 52.197) (width 0.25) (layer "F.Cu") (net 4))
 (segment (start 64.531 52.847) (end 63.627 52.847) (width 0.25) (layer "F.Cu") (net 10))
 (segment (start 65.8622 53.3147) (end 64.9987 53.3147) (width 0.25) (layer "F.Cu") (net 10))
 (segment (start 64.9987 53.3147) (end 64.531 52.847) (width 0.25) (layer "F.Cu") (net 10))
 (segment (start 57.24 61.5) (end 54.98 61.5) (width 0.25) (layer "F.Cu") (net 6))
 (segment (start 61.62 57.12) (end 57.24 61.5) (width 0.25) (layer "F.Cu") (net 6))
 (segment (start 68.453 58.49) (end 70.41 58.49) (width 0.25) (layer "F.Cu") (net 6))
 (segment (start 70.36 58.49) (end 70.37 58.5) (width 0.25) (layer "F.Cu") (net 6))
 (segment (start 70.41 58.49) (end 70.42 58.5) (width 0.25) (layer "F.Cu") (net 6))
 (segment (start 65.659 58.4708) (end 64.3082 57.12) (width 0.25) (layer "F.Cu") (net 6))
 (segment (start 70.31 58.49) (end 70.32 58.5) (width 0.25) (layer "F.Cu") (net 6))
 (segment (start 64.3082 57.12) (end 61.62 57.12) (width 0.25) (layer "F.Cu") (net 6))
 (via (at 68.453 58.49) (size 0.6) (drill 0.3) (layers "F.Cu" "B.Cu") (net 6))
 (via (at 65.659 58.4708) (size 0.6) (drill 0.3) (layers "F.Cu" "B.Cu") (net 6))
 (segment (start 68.453 58.49) (end 65.6782 58.49) (width 0.25) (layer "B.Cu") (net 6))
 (segment (start 65.6782 58.49) (end 65.659 58.4708) (width 0.25) (layer "B.Cu") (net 6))
 (segment (start 59.7916 57.2008) (end 59.7408 57.2008) (width 0.25) (layer "F.Cu") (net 5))
 (segment (start 68.472931 59.517669) (end 70.402331 59.517669) (width 0.25) (layer "F.Cu") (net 5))
 (segment (start 68.472931 59.517669) (end 68.4906 59.5) (width 0.25) (layer "F.Cu") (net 5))
 (segment (start 70.402331 59.517669) (end 70.42 59.5) (width 0.25) (layer "F.Cu") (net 5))
 (segment (start 59.7408 57.2008) (end 56.4416 60.5) (width 0.25) (layer "F.Cu") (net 5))
 (segment (start 56.4416 60.5) (end 54.98 60.5) (width 0.25) (layer "F.Cu") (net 5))
 (segment (start 68.472931 59.517669) (end 68.455262 59.5) (width 0.25) (layer "F.Cu") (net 5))
 (segment (start 70.352331 59.517669) (end 70.37 59.5) (width 0.25) (layer "F.Cu") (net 5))
 (via (at 59.7916 57.2008) (size 0.6) (drill 0.3) (layers "F.Cu" "B.Cu") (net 5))
 (via (at 68.472931 59.517669) (size 0.6) (drill 0.3) (layers "F.Cu" "B.Cu") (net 5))
 (segment (start 61.4492 57.2008) (end 59.7916 57.2008) (width 0.25) (layer "B.Cu") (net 5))
 (segment (start 68.472931 59.517669) (end 65.791469 59.517669) (width 0.25) (layer "B.Cu") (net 5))
 (segment (start 65.791469 59.517669) (end 63.4638 57.19) (width 0.25) (layer "B.Cu") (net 5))
 (segment (start 61.46 57.19) (end 61.4492 57.2008) (width 0.25) (layer "B.Cu") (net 5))
 (segment (start 63.4638 57.19) (end 61.46 57.19) (width 0.25) (layer "B.Cu") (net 5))
 (segment (start 63.627 54.4068) (end 63.1698 54.864) (width 0.25) (layer "F.Cu") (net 9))
 (segment (start 64.5202 65.881) (end 64.5202 66.081) (width 0.25) (layer "F.Cu") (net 9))
 (segment (start 62.8402 65.941) (end 62.8452 65.936) (width 0.25) (layer "F.Cu") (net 9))
 (segment (start 63.5452 65.936) (end 64.4652 65.936) (width 0.25) (layer "F.Cu") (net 9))
 (segment (start 61.6202 65.941) (end 60.4038 65.941) (width 0.25) (layer "F.Cu") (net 9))
 (segment (start 65.6082 68.5546) (end 65.1502 68.0966) (width 0.25) (layer "F.Cu") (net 9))
 (segment (start 58.55 65.1) (end 58.55 65.5858) (width 0.25) (layer "F.Cu") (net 9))
 (segment (start 62.8452 65.936) (end 63.5452 65.936) (width 0.25) (layer "F.Cu") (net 9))
 (segment (start 61.727 52.847) (end 62.1942 52.847) (width 0.25) (layer "F.Cu") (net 9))
 (segment (start 68.5546 68.5292) (end 65.6336 68.5292) (width 0.25) (layer "F.Cu") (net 9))
 (segment (start 65.1502 66.711) (end 65.1502 67.481) (width 0.25) (layer "F.Cu") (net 9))
 (segment (start 68.4754 54.6354) (end 68.83 54.99) (width 0.25) (layer "F.Cu") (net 9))
 (segment (start 63.627 53.497) (end 64.1396 53.497) (width 0.25) (layer "F.Cu") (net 9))
 (segment (start 65.278 54.6354) (end 68.4754 54.6354) (width 0.25) (layer "F.Cu") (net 9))
 (segment (start 62.1942 52.847) (end 62.8442 53.497) (width 0.25) (layer "F.Cu") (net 9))
 (segment (start 64.5202 66.081) (end 65.1502 66.711) (width 0.25) (layer "F.Cu") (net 9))
 (segment (start 61.6202 65.941) (end 62.8402 65.941) (width 0.25) (layer "F.Cu") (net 9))
 (segment (start 59.5628 65.1) (end 58.55 65.1) (width 0.25) (layer "F.Cu") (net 9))
 (segment (start 65.6336 68.5292) (end 65.6082 68.5546) (width 0.25) (layer "F.Cu") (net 9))
 (segment (start 63.627 53.497) (end 63.627 54.4068) (width 0.25) (layer "F.Cu") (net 9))
 (segment (start 64.1396 53.497) (end 65.278 54.6354) (width 0.25) (layer "F.Cu") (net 9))
 (segment (start 69.9008 67.183) (end 68.5546 68.5292) (width 0.25) (layer "F.Cu") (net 9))
 (segment (start 60.4038 65.941) (end 59.5628 65.1) (width 0.25) (layer "F.Cu") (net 9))
 (segment (start 69.9008 63.881) (end 69.9008 67.183) (width 0.25) (layer "F.Cu") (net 9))
 (segment (start 62.8442 53.497) (end 63.627 53.497) (width 0.25) (layer "F.Cu") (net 9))
 (segment (start 65.1502 68.0966) (end 65.1502 67.481) (width 0.25) (layer "F.Cu") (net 9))
 (segment (start 64.4652 65.936) (end 64.5202 65.881) (width 0.25) (layer "F.Cu") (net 9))
 (via (at 69.9008 63.881) (size 0.6) (drill 0.3) (layers "F.Cu" "B.Cu") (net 9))
 (via (at 68.83 54.99) (size 0.6) (drill 0.3) (layers "F.Cu" "B.Cu") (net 9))
 (segment (start 69.9008 56.0832) (end 68.83 55.0124) (width 0.25) (layer "B.Cu") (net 9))
 (segment (start 68.83 55.0124) (end 68.83 54.99) (width 0.25) (layer "B.Cu") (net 9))
 (segment (start 69.9008 63.881) (end 69.9008 56.0832) (width 0.25) (layer "B.Cu") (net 9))
 (segment (start 68.426 63.981) (end 68.4276 63.9826) (width 0.25) (layer "F.Cu") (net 1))
 (segment (start 66.802 61.9252) (end 66.802 63.3476) (width 0.25) (layer "F.Cu") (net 1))
 (segment (start 62.7 59.2125) (end 64.0893 59.2125) (width 0.25) (layer "F.Cu") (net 1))
 (segment (start 66.7952 63.981) (end 68.426 63.981) (width 0.25) (layer "F.Cu") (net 1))
 (segment (start 64.0893 59.2125) (end 66.802 61.9252) (width 0.25) (layer "F.Cu") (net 1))
 (segment (start 66.7952 63.3544) (end 66.7952 63.981) (width 0.25) (layer "F.Cu") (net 1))
 (segment (start 66.802 63.3476) (end 66.7952 63.3544) (width 0.25) (layer "F.Cu") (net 1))
 (segment (start 60.0375 60.7875) (end 62.7 60.7875) (width 0.25) (layer "F.Cu") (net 2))
 (segment (start 57.6 63.225) (end 57.6 62.56) (width 0.25) (layer "F.Cu") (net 2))
 (segment (start 57.6 63.225) (end 60.0375 60.7875) (width 0.25) (layer "F.Cu") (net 2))
 (segment (start 62.0058 63.225) (end 59.5 63.225) (width 0.25) (layer "F.Cu") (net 8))
 (segment (start 59.545 63.18) (end 59.5 63.225) (width 0.25) (layer "F.Cu") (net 8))
 (segment (start 64.5202 63.981) (end 62.7618 63.981) (width 0.25) (layer "F.Cu") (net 8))
 (segment (start 62.7618 63.981) (end 62.0058 63.225) (width 0.25) (layer "F.Cu") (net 8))
 (segment (start 66.7952 67.346) (end 66.6602 67.481) (width 0.25) (layer "F.Cu") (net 7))
 (segment (start 67.7164 67.3608) (end 68.4276 67.3608) (width 0.25) (layer "F.Cu") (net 7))
 (segment (start 66.7952 65.881) (end 66.7952 67.196) (width 0.25) (layer "F.Cu") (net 7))
 (segment (start 66.5226 67.481) (end 67.5962 67.481) (width 0.25) (layer "F.Cu") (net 7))
 (segment (start 66.5226 67.481) (end 66.1702 67.481) (width 0.25) (layer "F.Cu") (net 7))
 (segment (start 66.7952 67.196) (end 66.7952 67.346) (width 0.25) (layer "F.Cu") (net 7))
 (segment (start 66.6602 67.481) (end 66.5226 67.481) (width 0.25) (layer "F.Cu") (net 7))
 (segment (start 67.5962 67.481) (end 67.7164 67.3608) (width 0.25) (layer "F.Cu") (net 7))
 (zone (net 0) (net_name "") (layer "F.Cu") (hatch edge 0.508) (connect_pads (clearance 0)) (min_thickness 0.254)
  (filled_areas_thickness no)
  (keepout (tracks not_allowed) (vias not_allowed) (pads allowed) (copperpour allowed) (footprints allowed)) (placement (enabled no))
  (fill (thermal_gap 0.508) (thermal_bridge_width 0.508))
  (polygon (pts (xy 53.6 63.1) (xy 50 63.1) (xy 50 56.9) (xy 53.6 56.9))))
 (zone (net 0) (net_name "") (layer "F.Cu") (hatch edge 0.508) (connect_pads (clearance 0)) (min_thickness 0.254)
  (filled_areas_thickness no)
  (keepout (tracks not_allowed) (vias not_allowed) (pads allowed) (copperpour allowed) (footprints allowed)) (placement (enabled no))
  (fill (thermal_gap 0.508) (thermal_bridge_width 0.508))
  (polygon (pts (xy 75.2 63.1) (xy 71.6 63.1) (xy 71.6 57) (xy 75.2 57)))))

